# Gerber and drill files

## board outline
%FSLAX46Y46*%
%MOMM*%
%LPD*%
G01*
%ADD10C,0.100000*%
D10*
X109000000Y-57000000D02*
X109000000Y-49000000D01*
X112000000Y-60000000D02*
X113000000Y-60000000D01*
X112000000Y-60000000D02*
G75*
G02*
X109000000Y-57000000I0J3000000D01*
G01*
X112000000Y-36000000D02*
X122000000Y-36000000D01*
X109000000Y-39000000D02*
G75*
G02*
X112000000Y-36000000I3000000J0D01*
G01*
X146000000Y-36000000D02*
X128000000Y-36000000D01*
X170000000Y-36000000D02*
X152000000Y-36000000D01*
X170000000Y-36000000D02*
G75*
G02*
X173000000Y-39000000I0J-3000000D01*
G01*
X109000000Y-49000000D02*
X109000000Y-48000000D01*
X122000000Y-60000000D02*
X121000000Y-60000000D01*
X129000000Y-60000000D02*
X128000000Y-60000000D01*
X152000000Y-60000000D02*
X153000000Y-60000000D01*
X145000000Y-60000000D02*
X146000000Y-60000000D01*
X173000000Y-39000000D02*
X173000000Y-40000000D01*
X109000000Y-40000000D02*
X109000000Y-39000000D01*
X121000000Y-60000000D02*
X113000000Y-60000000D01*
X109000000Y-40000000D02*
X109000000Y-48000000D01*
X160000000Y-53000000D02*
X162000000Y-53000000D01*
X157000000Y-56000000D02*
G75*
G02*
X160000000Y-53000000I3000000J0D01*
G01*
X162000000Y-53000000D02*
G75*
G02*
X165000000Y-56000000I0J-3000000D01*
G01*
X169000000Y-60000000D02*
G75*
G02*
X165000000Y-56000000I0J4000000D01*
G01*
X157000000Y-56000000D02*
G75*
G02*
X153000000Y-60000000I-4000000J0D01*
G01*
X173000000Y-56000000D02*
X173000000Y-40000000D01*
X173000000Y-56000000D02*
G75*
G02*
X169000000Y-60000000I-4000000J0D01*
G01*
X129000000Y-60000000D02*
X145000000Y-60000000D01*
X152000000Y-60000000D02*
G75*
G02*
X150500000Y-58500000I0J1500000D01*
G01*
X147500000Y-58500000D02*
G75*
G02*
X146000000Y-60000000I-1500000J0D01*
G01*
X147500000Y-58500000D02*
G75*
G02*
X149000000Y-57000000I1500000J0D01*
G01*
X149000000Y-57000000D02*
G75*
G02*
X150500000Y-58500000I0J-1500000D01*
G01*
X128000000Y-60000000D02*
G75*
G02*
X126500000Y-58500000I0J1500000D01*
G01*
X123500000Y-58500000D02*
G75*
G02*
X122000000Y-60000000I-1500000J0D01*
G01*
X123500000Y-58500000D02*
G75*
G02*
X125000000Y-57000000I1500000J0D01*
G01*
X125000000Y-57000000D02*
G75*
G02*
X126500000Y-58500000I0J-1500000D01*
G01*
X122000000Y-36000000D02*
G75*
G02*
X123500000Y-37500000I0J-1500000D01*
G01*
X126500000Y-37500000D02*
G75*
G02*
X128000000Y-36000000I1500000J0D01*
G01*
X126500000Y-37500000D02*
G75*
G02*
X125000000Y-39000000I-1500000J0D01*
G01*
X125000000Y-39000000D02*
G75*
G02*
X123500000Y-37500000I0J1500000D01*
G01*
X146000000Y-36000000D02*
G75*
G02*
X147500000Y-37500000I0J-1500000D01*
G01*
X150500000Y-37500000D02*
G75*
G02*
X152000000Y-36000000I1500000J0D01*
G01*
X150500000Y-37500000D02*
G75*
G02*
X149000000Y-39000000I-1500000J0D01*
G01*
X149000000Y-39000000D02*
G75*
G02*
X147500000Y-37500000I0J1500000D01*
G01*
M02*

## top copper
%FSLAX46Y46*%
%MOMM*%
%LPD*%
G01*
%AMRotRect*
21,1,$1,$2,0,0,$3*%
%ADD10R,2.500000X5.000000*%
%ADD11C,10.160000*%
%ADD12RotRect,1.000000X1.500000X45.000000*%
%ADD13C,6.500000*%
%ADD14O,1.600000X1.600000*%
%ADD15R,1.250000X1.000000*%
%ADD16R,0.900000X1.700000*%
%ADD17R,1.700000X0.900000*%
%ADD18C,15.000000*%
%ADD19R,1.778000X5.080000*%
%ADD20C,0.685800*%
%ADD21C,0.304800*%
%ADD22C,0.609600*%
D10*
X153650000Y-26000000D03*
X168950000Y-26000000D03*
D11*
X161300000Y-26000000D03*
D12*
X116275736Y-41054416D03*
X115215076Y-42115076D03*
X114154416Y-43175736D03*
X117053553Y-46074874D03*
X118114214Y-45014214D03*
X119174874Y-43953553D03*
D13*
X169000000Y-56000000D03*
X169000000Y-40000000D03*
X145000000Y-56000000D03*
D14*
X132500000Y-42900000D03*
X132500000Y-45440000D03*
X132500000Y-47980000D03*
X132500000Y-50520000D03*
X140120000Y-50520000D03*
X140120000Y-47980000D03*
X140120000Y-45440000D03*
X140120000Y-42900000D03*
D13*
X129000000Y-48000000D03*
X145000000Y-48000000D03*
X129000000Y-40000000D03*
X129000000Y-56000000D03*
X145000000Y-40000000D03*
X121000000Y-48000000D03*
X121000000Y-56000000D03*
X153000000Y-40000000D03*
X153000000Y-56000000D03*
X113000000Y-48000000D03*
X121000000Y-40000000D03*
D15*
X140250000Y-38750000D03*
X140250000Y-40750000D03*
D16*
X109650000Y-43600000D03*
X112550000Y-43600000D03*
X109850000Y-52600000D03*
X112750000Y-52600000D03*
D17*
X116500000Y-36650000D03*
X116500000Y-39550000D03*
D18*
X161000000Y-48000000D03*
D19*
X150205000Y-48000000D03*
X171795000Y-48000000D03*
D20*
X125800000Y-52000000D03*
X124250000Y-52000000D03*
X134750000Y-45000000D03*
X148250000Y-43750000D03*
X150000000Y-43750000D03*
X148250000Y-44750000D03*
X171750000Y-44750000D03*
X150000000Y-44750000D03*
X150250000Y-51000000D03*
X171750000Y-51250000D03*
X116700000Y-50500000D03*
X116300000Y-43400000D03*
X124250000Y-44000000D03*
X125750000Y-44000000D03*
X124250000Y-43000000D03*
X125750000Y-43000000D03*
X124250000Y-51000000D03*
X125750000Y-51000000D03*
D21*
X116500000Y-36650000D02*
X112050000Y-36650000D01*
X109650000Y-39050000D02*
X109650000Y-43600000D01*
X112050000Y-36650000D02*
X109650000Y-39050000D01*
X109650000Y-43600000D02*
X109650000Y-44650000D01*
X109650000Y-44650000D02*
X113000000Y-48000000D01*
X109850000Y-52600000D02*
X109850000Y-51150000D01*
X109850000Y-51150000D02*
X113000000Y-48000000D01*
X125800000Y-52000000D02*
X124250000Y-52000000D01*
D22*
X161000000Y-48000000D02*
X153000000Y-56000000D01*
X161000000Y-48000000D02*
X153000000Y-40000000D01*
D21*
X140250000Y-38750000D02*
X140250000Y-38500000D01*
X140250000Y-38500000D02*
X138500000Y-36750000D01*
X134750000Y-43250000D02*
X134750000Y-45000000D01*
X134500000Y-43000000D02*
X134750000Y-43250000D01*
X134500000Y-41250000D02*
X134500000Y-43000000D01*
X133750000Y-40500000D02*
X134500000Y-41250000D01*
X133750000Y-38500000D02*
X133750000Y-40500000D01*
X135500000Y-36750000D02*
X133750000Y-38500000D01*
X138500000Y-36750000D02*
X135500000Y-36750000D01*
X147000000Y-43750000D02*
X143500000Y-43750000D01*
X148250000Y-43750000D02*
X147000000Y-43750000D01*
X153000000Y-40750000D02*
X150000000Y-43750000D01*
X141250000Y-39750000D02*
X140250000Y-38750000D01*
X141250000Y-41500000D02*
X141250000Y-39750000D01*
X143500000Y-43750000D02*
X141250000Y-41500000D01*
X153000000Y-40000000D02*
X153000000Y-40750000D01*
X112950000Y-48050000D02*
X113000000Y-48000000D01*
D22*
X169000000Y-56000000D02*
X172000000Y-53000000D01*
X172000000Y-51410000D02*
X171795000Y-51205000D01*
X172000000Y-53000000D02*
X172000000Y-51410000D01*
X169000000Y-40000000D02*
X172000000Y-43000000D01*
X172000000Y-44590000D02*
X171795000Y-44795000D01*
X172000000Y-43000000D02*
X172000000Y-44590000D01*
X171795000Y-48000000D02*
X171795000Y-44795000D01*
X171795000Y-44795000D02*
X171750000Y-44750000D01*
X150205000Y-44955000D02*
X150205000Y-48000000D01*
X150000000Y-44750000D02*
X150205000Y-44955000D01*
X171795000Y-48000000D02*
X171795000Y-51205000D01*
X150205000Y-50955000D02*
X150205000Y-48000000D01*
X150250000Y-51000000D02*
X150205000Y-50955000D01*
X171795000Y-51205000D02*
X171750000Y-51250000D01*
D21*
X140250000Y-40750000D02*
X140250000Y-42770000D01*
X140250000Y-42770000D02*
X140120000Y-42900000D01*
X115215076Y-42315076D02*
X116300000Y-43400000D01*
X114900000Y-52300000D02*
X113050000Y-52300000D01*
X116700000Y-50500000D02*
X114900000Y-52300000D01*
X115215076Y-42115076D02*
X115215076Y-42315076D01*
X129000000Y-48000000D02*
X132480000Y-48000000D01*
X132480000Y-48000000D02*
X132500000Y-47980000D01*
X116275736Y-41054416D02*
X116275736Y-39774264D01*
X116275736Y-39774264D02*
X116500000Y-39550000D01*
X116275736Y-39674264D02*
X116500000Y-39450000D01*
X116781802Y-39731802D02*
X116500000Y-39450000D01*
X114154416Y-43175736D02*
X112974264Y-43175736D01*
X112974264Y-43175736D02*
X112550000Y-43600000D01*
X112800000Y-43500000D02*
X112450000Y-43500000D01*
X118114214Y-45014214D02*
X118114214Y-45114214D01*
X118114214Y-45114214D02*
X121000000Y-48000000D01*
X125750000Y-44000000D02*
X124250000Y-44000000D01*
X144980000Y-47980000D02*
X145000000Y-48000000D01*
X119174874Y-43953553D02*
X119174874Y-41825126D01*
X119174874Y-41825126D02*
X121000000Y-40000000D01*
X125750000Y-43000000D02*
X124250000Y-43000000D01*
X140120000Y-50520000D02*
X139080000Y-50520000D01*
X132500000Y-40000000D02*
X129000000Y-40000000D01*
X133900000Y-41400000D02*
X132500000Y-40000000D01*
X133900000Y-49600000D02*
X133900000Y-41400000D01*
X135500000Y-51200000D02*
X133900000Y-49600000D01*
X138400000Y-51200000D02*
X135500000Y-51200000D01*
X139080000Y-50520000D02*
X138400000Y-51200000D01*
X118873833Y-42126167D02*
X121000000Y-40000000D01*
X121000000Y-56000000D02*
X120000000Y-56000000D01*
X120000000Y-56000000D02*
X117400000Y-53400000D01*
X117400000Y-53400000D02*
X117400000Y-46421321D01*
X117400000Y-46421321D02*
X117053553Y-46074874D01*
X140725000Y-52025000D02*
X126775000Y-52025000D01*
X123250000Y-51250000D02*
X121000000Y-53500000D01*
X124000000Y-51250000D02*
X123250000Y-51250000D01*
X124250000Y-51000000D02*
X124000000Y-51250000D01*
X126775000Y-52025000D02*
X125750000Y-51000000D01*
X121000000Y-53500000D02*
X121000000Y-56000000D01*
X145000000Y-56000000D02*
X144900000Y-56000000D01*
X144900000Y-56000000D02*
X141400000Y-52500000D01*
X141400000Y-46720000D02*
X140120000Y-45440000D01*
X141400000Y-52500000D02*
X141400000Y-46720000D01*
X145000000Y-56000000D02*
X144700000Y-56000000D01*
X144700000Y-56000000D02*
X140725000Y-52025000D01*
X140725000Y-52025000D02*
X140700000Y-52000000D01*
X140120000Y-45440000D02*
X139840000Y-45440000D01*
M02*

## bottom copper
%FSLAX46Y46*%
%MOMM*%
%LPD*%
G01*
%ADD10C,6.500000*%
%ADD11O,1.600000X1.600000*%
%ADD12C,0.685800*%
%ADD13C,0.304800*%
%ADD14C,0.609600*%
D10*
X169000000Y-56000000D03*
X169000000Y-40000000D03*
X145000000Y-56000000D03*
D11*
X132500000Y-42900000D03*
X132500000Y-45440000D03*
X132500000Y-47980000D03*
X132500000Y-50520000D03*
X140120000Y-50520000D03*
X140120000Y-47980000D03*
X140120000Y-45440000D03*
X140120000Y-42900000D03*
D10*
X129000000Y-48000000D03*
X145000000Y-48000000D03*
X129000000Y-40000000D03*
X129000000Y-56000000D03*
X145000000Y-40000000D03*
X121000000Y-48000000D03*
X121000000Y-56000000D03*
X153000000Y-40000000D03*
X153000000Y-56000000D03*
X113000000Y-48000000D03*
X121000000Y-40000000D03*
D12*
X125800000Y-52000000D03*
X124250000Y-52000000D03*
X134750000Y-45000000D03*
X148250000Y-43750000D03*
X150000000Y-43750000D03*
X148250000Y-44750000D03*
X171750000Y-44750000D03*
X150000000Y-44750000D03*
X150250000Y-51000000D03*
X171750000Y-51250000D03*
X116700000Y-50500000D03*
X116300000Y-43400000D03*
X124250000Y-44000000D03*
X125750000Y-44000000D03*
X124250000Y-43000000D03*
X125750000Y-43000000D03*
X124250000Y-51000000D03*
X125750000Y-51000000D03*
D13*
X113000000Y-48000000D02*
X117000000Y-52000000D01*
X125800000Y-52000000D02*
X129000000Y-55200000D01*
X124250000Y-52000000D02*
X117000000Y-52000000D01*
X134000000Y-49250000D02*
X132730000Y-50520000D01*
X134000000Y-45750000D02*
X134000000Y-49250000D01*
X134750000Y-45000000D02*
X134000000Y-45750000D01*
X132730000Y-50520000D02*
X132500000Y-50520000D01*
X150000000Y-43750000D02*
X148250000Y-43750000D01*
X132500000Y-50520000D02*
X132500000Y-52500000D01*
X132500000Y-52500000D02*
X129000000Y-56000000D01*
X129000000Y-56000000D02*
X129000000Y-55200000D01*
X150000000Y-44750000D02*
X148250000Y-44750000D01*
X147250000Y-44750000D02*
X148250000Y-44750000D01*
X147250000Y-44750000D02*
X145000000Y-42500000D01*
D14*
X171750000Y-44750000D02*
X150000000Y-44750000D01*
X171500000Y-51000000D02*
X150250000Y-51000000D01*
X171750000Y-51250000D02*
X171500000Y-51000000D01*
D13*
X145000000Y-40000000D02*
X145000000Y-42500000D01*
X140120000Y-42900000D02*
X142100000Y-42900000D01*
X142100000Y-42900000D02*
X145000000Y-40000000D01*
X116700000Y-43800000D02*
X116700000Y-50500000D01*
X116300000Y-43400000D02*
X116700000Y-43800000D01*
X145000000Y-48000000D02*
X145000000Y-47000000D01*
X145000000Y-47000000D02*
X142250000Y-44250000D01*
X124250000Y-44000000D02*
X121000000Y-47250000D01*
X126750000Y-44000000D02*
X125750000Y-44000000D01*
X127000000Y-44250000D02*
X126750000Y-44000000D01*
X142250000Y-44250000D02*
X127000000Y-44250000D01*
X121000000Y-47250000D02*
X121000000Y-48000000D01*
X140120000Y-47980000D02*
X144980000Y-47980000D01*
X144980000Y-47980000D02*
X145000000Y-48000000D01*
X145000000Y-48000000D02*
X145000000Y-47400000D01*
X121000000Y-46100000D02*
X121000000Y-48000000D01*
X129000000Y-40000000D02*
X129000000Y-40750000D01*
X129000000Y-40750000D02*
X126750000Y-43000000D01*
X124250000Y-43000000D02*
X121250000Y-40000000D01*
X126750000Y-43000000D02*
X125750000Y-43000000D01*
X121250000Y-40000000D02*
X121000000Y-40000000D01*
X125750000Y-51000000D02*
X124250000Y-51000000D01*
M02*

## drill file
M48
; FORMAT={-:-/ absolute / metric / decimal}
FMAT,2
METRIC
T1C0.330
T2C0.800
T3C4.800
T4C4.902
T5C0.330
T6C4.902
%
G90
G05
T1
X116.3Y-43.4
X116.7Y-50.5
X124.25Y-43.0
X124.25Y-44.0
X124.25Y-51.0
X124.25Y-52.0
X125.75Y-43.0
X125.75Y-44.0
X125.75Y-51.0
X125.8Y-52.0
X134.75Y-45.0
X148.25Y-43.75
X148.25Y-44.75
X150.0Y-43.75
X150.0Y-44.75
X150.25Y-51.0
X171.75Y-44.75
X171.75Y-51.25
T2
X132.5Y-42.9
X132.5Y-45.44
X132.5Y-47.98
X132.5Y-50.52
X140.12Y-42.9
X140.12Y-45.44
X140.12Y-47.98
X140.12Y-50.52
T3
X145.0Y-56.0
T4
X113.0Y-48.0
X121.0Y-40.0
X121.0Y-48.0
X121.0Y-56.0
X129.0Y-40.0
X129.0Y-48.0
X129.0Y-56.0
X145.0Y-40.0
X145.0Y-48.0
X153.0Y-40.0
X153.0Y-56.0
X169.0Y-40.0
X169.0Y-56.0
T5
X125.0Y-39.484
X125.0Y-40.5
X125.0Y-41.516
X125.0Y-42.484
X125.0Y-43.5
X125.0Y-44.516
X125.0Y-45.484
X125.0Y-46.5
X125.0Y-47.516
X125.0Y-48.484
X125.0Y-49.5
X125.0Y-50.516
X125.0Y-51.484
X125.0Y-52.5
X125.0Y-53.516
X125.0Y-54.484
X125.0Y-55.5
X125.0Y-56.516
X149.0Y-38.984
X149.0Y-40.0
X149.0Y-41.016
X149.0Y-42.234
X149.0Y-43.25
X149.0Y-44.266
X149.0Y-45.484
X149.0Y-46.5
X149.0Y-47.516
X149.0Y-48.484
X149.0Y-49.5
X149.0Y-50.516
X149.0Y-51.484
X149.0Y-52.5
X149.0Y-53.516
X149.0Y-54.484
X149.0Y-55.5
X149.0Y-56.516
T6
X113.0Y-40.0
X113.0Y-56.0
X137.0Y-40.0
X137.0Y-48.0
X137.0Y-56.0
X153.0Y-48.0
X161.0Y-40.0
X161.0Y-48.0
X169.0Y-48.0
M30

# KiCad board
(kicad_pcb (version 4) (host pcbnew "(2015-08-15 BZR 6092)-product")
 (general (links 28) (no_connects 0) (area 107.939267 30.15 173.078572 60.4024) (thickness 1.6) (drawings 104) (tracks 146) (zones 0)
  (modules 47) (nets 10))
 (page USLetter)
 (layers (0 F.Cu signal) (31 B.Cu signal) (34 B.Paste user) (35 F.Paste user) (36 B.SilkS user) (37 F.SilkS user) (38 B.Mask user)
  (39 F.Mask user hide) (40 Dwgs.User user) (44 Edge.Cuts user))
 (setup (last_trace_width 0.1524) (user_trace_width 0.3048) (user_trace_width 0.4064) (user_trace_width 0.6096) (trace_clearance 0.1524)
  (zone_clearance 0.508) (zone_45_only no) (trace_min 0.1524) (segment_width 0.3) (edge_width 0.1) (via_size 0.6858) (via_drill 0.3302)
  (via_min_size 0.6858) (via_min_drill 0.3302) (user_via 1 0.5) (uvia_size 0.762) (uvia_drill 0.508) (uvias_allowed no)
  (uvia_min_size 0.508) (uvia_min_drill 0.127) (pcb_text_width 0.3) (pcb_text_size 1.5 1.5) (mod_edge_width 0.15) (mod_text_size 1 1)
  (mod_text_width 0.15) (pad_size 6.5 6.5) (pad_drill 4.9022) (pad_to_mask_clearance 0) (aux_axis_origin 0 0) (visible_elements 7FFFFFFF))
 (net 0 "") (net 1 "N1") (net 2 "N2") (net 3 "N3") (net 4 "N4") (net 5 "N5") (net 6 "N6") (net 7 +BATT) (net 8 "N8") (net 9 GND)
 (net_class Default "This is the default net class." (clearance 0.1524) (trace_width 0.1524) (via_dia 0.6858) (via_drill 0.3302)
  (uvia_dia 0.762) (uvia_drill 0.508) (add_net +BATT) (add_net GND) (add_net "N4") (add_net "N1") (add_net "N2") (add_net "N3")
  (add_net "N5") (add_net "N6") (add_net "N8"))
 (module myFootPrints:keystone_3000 (layer F.Cu) (at 161.3 26)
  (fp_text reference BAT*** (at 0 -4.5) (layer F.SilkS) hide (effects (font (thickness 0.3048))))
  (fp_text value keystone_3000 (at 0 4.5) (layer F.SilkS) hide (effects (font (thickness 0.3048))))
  (pad 1 smd rect (at -7.65 0) (size 2.5 5) (layers F.Cu F.Paste F.Mask))
  (pad 1 smd rect (at 7.65 0) (size 2.5 5) (layers F.Cu F.Paste F.Mask))
  (pad 2 smd circle (at 0 0) (size 10.16 10.16) (layers F.Cu F.Paste F.Mask)))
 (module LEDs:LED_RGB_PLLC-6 (layer F.Cu) (at 116.7 43.6 315)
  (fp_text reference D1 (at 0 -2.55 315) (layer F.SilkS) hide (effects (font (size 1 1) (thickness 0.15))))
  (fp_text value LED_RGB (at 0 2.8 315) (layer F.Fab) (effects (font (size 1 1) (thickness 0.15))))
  (pad 1 smd rect (at -2.1 -1.5 45) (size 1 1.5) (layers F.Cu F.Paste F.Mask) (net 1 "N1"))
  (pad 2 smd rect (at -2.1 0 45) (size 1 1.5) (layers F.Cu F.Paste F.Mask) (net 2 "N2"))
  (pad 3 smd rect (at -2.1 1.5 45) (size 1 1.5) (layers F.Cu F.Paste F.Mask) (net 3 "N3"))
  (pad 4 smd rect (at 2 1.5 45) (size 1 1.5) (layers F.Cu F.Paste F.Mask) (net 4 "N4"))
  (pad 5 smd rect (at 2 0 45) (size 1 1.5) (layers F.Cu F.Paste F.Mask) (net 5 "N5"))
  (pad 6 smd rect (at 2 -1.5 45) (size 1 1.5) (layers F.Cu F.Paste F.Mask) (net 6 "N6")))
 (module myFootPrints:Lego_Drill (layer F.Cu) (at 113 40)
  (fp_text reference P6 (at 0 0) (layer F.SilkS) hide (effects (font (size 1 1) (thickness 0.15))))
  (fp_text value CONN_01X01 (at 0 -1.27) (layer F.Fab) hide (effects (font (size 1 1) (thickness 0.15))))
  (pad "" np_thru_hole circle (at 0 0) (size 4.9022 4.9022) (drill 4.9022) (layers *.Cu *.Mask F.SilkS)))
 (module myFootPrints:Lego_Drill (layer F.Cu) (at 113 56)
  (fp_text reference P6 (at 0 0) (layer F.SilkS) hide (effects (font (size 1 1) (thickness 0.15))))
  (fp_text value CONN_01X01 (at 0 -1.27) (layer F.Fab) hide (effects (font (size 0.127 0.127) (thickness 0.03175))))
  (pad "" np_thru_hole circle (at 0 0) (size 4.9022 4.9022) (drill 4.9022) (layers *.Cu *.Mask F.SilkS)))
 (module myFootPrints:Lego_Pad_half (layer F.Cu) (at 169 56 180)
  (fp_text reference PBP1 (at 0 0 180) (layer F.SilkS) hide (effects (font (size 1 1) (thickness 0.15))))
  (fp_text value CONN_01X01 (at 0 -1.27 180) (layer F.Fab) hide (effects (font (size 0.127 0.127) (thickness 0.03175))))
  (pad 1 thru_hole circle (at 0 0 180) (size 6.5 6.5) (drill 4.9022) (layers *.Cu B.Mask) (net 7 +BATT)))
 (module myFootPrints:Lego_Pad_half (layer F.Cu) (at 169 40 270)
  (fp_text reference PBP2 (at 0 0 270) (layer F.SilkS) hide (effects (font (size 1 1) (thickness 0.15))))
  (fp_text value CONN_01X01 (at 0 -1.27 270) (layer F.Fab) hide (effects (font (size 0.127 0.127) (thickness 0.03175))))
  (pad 1 thru_hole circle (at 0 0 270) (size 6.5 6.5) (drill 4.9022) (layers *.Cu B.Mask) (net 7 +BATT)))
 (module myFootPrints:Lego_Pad (layer F.Cu) (at 145 56)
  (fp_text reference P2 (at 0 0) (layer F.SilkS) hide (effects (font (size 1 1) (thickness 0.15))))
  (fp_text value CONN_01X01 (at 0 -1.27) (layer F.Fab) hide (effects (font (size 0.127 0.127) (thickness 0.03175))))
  (pad 1 thru_hole circle (at 0 0) (size 6.5 6.5) (drill 4.8) (layers *.Cu *.Mask F.SilkS) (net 4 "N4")))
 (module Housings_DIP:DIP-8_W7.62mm (layer F.Cu) (at 132.5 42.9)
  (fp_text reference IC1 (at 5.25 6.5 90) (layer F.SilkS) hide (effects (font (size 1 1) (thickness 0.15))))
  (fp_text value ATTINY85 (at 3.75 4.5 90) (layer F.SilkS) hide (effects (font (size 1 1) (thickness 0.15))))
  (pad 1 thru_hole oval (at 0 0) (size 1.6 1.6) (drill 0.8) (layers *.Cu *.Mask F.SilkS))
  (pad 2 thru_hole oval (at 0 2.54) (size 1.6 1.6) (drill 0.8) (layers *.Cu *.Mask F.SilkS))
  (pad 3 thru_hole oval (at 0 5.08) (size 1.6 1.6) (drill 0.8) (layers *.Cu *.Mask F.SilkS) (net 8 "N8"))
  (pad 4 thru_hole oval (at 0 7.62) (size 1.6 1.6) (drill 0.8) (layers *.Cu *.Mask F.SilkS) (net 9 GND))
  (pad 5 thru_hole oval (at 7.62 7.62) (size 1.6 1.6) (drill 0.8) (layers *.Cu *.Mask F.SilkS) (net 6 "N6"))
  (pad 6 thru_hole oval (at 7.62 5.08) (size 1.6 1.6) (drill 0.8) (layers *.Cu *.Mask F.SilkS) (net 5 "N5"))
  (pad 7 thru_hole oval (at 7.62 2.54) (size 1.6 1.6) (drill 0.8) (layers *.Cu *.Mask F.SilkS) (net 4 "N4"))
  (pad 8 thru_hole oval (at 7.62 0) (size 1.6 1.6) (drill 0.8) (layers *.Cu *.Mask F.SilkS) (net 7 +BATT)))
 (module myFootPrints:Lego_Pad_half (layer F.Cu) (at 129 48 45)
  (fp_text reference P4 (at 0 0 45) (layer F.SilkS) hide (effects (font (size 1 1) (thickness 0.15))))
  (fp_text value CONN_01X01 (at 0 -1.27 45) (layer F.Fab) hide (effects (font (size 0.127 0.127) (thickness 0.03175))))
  (pad 1 thru_hole circle (at 0 0 45) (size 6.5 6.5) (drill 4.9022) (layers *.Cu *.Mask F.SilkS) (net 8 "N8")))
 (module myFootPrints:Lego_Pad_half (layer F.Cu) (at 145 48 225)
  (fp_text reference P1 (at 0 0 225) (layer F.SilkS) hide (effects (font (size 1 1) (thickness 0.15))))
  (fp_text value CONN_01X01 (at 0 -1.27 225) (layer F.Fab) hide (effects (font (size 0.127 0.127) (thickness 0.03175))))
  (pad 1 thru_hole circle (at 0 0 225) (size 6.5 6.5) (drill 4.9022) (layers *.Cu *.Mask F.SilkS) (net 5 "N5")))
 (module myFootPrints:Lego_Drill (layer F.Cu) (at 137 40)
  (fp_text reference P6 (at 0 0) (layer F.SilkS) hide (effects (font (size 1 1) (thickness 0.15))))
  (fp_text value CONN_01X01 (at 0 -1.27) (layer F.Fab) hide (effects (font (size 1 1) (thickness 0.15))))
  (pad "" np_thru_hole circle (at 0 0) (size 4.9022 4.9022) (drill 4.9022) (layers *.Cu *.Mask F.SilkS)))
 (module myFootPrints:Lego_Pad (layer F.Cu) (at 129 40)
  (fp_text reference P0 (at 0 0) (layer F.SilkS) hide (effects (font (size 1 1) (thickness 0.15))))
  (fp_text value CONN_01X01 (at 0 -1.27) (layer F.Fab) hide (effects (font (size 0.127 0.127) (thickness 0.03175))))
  (pad 1 thru_hole circle (at 0 0) (size 6.5 6.5) (drill 4.9022) (layers *.Cu *.Mask F.SilkS) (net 6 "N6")))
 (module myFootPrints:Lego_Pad (layer F.Cu) (at 129 56)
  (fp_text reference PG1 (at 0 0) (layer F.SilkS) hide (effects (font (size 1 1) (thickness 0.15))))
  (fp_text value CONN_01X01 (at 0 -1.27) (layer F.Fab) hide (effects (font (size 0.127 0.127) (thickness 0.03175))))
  (pad 1 thru_hole circle (at 0 0) (size 6.5 6.5) (drill 4.9022) (layers *.Cu *.Mask F.SilkS) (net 9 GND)))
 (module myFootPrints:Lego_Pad (layer F.Cu) (at 145 40)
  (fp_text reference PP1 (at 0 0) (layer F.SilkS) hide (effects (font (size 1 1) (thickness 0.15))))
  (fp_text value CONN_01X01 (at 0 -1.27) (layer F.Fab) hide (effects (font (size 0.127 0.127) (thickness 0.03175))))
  (pad 1 thru_hole circle (at 0 0) (size 6.5 6.5) (drill 4.9022) (layers *.Cu *.Mask F.SilkS) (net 7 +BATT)))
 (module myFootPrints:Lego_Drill (layer F.Cu) (at 137 48)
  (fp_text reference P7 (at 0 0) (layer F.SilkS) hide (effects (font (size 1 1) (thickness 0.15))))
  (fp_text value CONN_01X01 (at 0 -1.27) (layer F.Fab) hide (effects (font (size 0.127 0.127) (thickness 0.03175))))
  (pad "" np_thru_hole circle (at 0 0) (size 4.9022 4.9022) (drill 4.9022) (layers *.Cu *.Mask F.SilkS)))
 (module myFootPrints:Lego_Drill (layer F.Cu) (at 137 56)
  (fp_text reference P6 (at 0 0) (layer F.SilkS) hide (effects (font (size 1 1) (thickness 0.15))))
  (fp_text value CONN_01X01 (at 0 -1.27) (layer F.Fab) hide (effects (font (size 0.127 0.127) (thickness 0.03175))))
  (pad "" np_thru_hole circle (at 0 0) (size 4.9022 4.9022) (drill 4.9022) (layers *.Cu *.Mask F.SilkS)))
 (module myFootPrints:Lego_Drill (layer F.Cu) (at 161 48)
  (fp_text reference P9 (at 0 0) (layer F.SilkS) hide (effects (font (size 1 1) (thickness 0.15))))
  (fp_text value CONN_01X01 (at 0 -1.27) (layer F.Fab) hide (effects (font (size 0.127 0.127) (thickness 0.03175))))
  (pad "" np_thru_hole circle (at 0 0) (size 4.9022 4.9022) (drill 4.9022) (layers *.Cu *.Mask F.SilkS)))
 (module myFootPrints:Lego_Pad (layer F.Cu) (at 121 48)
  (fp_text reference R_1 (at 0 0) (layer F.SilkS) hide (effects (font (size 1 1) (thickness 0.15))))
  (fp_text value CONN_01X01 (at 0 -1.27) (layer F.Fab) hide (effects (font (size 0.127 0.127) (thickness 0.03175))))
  (pad 1 thru_hole circle (at 0 0) (size 6.5 6.5) (drill 4.9022) (layers *.Cu *.Mask F.SilkS) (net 5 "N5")))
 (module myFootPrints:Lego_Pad (layer F.Cu) (at 121 56)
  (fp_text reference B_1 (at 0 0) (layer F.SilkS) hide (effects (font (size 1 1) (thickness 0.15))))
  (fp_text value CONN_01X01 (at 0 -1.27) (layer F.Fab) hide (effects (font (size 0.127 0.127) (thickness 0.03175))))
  (pad 1 thru_hole circle (at 0 0) (size 6.5 6.5) (drill 4.9022) (layers *.Cu *.Mask F.SilkS) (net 4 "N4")))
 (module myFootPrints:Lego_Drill (layer F.Cu) (at 169 48)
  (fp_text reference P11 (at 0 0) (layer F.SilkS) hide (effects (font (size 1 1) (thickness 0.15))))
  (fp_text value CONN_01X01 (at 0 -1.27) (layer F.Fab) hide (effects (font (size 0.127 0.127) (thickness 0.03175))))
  (pad "" np_thru_hole circle (at 0 0) (size 4.9022 4.9022) (drill 4.9022) (layers *.Cu *.Mask F.SilkS)))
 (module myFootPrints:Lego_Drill (layer F.Cu) (at 153 48)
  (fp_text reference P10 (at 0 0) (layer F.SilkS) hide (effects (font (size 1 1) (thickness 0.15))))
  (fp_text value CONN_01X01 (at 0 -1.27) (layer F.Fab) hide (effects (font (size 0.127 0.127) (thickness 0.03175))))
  (pad "" np_thru_hole circle (at 0 0) (size 4.9022 4.9022) (drill 4.9022) (layers *.Cu *.Mask F.SilkS)))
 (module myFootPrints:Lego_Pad (layer F.Cu) (at 153 40)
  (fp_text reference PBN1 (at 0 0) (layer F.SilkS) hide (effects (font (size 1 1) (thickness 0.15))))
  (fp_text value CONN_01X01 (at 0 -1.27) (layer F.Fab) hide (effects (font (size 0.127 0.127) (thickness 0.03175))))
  (pad 1 thru_hole circle (at 0 0) (size 6.5 6.5) (drill 4.9022) (layers *.Cu *.Mask F.SilkS) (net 9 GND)))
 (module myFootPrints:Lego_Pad (layer F.Cu) (at 153 56)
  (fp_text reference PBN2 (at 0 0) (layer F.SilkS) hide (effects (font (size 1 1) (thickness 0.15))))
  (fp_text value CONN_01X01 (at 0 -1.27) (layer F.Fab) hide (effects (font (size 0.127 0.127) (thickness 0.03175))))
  (pad 1 thru_hole circle (at 0 0) (size 6.5 6.5) (drill 4.9022) (layers *.Cu *.Mask F.SilkS) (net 9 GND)))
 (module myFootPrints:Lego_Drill (layer F.Cu) (at 161 40)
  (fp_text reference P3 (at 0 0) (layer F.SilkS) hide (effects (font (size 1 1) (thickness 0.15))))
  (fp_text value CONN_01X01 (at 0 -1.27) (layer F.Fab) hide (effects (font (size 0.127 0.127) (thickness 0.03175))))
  (pad "" np_thru_hole circle (at 0 0) (size 4.9022 4.9022) (drill 4.9022) (layers *.Cu *.Mask F.SilkS)))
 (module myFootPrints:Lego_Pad (layer F.Cu) (at 113 48)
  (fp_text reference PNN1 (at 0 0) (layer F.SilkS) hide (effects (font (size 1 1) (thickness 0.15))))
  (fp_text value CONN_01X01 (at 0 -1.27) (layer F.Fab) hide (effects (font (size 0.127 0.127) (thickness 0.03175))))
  (pad 1 thru_hole circle (at 0 0) (size 6.5 6.5) (drill 4.9022) (layers *.Cu *.Mask F.SilkS) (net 9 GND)))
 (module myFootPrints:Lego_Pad (layer F.Cu) (at 121 40)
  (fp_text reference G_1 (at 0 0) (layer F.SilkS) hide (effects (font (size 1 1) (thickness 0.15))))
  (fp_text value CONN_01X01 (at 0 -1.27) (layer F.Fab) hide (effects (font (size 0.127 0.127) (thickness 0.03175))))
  (pad 1 thru_hole circle (at 0 0) (size 6.5 6.5) (drill 4.9022) (layers *.Cu *.Mask F.SilkS) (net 6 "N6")))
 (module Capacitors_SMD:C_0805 (layer F.Cu) (at 140.25 39.75 270)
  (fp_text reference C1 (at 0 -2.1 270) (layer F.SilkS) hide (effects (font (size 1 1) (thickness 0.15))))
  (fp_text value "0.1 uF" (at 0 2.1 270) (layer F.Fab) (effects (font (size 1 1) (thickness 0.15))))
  (pad 1 smd rect (at -1 0 270) (size 1 1.25) (layers F.Cu F.Paste F.Mask) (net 9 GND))
  (pad 2 smd rect (at 1 0 270) (size 1 1.25) (layers F.Cu F.Paste F.Mask) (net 7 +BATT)))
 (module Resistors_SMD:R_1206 (layer F.Cu) (at 111.1 43.6)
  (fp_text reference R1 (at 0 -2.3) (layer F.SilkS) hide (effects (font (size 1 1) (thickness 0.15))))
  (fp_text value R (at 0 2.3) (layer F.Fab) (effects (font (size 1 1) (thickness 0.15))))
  (pad 1 smd rect (at -1.45 0) (size 0.9 1.7) (layers F.Cu F.Paste F.Mask) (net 9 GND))
  (pad 2 smd rect (at 1.45 0) (size 0.9 1.7) (layers F.Cu F.Paste F.Mask) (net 3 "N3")))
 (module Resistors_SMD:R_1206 (layer F.Cu) (at 111.3 52.6)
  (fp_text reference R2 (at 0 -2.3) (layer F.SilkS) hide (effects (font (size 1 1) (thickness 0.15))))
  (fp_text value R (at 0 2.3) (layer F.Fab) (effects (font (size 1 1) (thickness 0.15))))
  (pad 1 smd rect (at -1.45 0) (size 0.9 1.7) (layers F.Cu F.Paste F.Mask) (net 9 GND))
  (pad 2 smd rect (at 1.45 0) (size 0.9 1.7) (layers F.Cu F.Paste F.Mask) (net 2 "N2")))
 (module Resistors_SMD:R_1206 (layer F.Cu) (at 116.5 38.1 270)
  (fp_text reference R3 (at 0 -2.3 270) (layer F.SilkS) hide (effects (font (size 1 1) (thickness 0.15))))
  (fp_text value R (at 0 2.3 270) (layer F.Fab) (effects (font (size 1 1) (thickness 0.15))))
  (pad 1 smd rect (at -1.45 0 270) (size 0.9 1.7) (layers F.Cu F.Paste F.Mask) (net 9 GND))
  (pad 2 smd rect (at 1.45 0 270) (size 0.9 1.7) (layers F.Cu F.Paste F.Mask) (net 1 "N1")))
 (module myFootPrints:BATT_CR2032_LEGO (layer F.Cu) (at 161 48)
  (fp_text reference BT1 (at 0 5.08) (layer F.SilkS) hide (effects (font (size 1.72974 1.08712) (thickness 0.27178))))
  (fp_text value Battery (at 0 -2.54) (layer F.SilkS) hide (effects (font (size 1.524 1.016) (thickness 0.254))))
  (pad 2 smd circle (at 0 0) (size 15 15) (layers F.Cu F.Paste F.Mask) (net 9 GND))
  (pad 1 smd rect (at -10.795 0) (size 1.778 5.08) (layers F.Cu F.Paste F.Mask) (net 7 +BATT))
  (pad 1 smd rect (at 10.795 0) (size 1.778 5.08) (layers F.Cu F.Paste F.Mask) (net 7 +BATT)))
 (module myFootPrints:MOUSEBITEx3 (layer F.Cu) (at 149 40 90)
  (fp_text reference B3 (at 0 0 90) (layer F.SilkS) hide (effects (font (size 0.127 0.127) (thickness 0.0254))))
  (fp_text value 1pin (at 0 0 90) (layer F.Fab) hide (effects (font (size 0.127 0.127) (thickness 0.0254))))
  (pad "" np_thru_hole circle (at -1.016 0 90) (size 0.3302 0.3302) (drill 0.3302) (layers *.Cu *.Mask F.SilkS))
  (pad "" np_thru_hole circle (at 1.016 0 90) (size 0.3302 0.3302) (drill 0.3302) (layers *.Cu *.Mask F.SilkS))
  (pad "" np_thru_hole circle (at 0 0 90) (size 0.3302 0.3302) (drill 0.3302) (layers *.Cu *.Mask F.SilkS)))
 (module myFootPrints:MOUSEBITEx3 (layer F.Cu) (at 149 49.5 90)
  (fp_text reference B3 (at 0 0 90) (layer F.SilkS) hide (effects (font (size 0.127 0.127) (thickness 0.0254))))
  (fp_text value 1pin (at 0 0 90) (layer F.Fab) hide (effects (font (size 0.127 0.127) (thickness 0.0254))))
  (pad "" np_thru_hole circle (at -1.016 0 90) (size 0.3302 0.3302) (drill 0.3302) (layers *.Cu *.Mask F.SilkS))
  (pad "" np_thru_hole circle (at 1.016 0 90) (size 0.3302 0.3302) (drill 0.3302) (layers *.Cu *.Mask F.SilkS))
  (pad "" np_thru_hole circle (at 0 0 90) (size 0.3302 0.3302) (drill 0.3302) (layers *.Cu *.Mask F.SilkS)))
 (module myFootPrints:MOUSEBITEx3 (layer F.Cu) (at 149 52.5 90)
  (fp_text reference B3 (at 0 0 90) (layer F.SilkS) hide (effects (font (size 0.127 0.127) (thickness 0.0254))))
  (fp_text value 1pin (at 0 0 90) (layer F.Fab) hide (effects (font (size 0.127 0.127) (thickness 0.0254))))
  (pad "" np_thru_hole circle (at -1.016 0 90) (size 0.3302 0.3302) (drill 0.3302) (layers *.Cu *.Mask F.SilkS))
  (pad "" np_thru_hole circle (at 1.016 0 90) (size 0.3302 0.3302) (drill 0.3302) (layers *.Cu *.Mask F.SilkS))
  (pad "" np_thru_hole circle (at 0 0 90) (size 0.3302 0.3302) (drill 0.3302) (layers *.Cu *.Mask F.SilkS)))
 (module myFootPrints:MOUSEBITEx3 (layer F.Cu) (at 149 55.5 90)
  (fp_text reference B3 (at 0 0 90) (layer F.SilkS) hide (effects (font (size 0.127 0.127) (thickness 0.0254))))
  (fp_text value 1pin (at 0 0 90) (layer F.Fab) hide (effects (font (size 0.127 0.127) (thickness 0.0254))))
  (pad "" np_thru_hole circle (at -1.016 0 90) (size 0.3302 0.3302) (drill 0.3302) (layers *.Cu *.Mask F.SilkS))
  (pad "" np_thru_hole circle (at 1.016 0 90) (size 0.3302 0.3302) (drill 0.3302) (layers *.Cu *.Mask F.SilkS))
  (pad "" np_thru_hole circle (at 0 0 90) (size 0.3302 0.3302) (drill 0.3302) (layers *.Cu *.Mask F.SilkS)))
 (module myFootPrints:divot (layer F.Cu) (at 149 60 180)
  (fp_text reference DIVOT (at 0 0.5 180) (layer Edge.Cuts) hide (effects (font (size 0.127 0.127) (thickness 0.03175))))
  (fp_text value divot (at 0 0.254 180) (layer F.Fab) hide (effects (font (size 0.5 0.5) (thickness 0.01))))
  (fp_arc (start -3 1.5) (end -3 0) (angle 90) (layer Edge.Cuts) (width 0.1))
  (fp_arc (start 3 1.5) (end 1.5 1.5) (angle 90) (layer Edge.Cuts) (width 0.1))
  (fp_arc (start 0 1.5) (end 1.5 1.5) (angle 90) (layer Edge.Cuts) (width 0.1))
  (fp_arc (start 0 1.5) (end 0 3) (angle 90) (layer Edge.Cuts) (width 0.1)))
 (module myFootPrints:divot (layer F.Cu) (at 125 60 180)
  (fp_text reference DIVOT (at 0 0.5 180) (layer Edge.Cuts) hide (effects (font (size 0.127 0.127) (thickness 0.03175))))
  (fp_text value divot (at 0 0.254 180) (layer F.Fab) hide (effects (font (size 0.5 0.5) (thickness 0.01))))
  (fp_arc (start -3 1.5) (end -3 0) (angle 90) (layer Edge.Cuts) (width 0.1))
  (fp_arc (start 3 1.5) (end 1.5 1.5) (angle 90) (layer Edge.Cuts) (width 0.1))
  (fp_arc (start 0 1.5) (end 1.5 1.5) (angle 90) (layer Edge.Cuts) (width 0.1))
  (fp_arc (start 0 1.5) (end 0 3) (angle 90) (layer Edge.Cuts) (width 0.1)))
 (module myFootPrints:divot (layer F.Cu) (at 125 36)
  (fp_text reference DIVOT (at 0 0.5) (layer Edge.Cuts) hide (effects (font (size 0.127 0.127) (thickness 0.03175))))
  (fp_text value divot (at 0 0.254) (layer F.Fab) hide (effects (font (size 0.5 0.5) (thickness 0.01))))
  (fp_arc (start -3 1.5) (end -3 0) (angle 90) (layer Edge.Cuts) (width 0.1))
  (fp_arc (start 3 1.5) (end 1.5 1.5) (angle 90) (layer Edge.Cuts) (width 0.1))
  (fp_arc (start 0 1.5) (end 1.5 1.5) (angle 90) (layer Edge.Cuts) (width 0.1))
  (fp_arc (start 0 1.5) (end 0 3) (angle 90) (layer Edge.Cuts) (width 0.1)))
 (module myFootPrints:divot (layer F.Cu) (at 149 36)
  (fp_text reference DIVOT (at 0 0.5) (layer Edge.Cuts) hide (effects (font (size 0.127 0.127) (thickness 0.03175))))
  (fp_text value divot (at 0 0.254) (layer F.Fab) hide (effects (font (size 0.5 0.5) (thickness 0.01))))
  (fp_arc (start -3 1.5) (end -3 0) (angle 90) (layer Edge.Cuts) (width 0.1))
  (fp_arc (start 3 1.5) (end 1.5 1.5) (angle 90) (layer Edge.Cuts) (width 0.1))
  (fp_arc (start 0 1.5) (end 1.5 1.5) (angle 90) (layer Edge.Cuts) (width 0.1))
  (fp_arc (start 0 1.5) (end 0 3) (angle 90) (layer Edge.Cuts) (width 0.1)))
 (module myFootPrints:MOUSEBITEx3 (layer F.Cu) (at 149 46.5 90)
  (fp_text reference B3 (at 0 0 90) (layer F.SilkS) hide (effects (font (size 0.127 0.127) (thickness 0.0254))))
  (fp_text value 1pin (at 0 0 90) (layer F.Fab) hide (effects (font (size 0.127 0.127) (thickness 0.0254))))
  (pad "" np_thru_hole circle (at -1.016 0 90) (size 0.3302 0.3302) (drill 0.3302) (layers *.Cu *.Mask F.SilkS))
  (pad "" np_thru_hole circle (at 1.016 0 90) (size 0.3302 0.3302) (drill 0.3302) (layers *.Cu *.Mask F.SilkS))
  (pad "" np_thru_hole circle (at 0 0 90) (size 0.3302 0.3302) (drill 0.3302) (layers *.Cu *.Mask F.SilkS)))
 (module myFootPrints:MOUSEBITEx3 (layer F.Cu) (at 149 43.25 90)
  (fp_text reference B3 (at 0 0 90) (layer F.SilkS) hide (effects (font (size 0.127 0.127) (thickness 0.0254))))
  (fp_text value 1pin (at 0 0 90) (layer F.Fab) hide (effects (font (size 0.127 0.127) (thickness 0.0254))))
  (pad "" np_thru_hole circle (at -1.016 0 90) (size 0.3302 0.3302) (drill 0.3302) (layers *.Cu *.Mask F.SilkS))
  (pad "" np_thru_hole circle (at 1.016 0 90) (size 0.3302 0.3302) (drill 0.3302) (layers *.Cu *.Mask F.SilkS))
  (pad "" np_thru_hole circle (at 0 0 90) (size 0.3302 0.3302) (drill 0.3302) (layers *.Cu *.Mask F.SilkS)))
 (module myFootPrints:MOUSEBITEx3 (layer F.Cu) (at 125 55.5 90)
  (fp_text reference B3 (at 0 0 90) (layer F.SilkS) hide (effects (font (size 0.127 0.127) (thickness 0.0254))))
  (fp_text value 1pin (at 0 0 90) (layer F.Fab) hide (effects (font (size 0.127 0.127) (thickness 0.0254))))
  (pad "" np_thru_hole circle (at -1.016 0 90) (size 0.3302 0.3302) (drill 0.3302) (layers *.Cu *.Mask F.SilkS))
  (pad "" np_thru_hole circle (at 1.016 0 90) (size 0.3302 0.3302) (drill 0.3302) (layers *.Cu *.Mask F.SilkS))
  (pad "" np_thru_hole circle (at 0 0 90) (size 0.3302 0.3302) (drill 0.3302) (layers *.Cu *.Mask F.SilkS)))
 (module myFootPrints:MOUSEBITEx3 (layer F.Cu) (at 125 52.5 90)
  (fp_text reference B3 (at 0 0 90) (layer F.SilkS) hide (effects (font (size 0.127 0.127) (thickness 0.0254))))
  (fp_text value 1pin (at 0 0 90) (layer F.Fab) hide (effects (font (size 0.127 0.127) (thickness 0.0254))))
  (pad "" np_thru_hole circle (at -1.016 0 90) (size 0.3302 0.3302) (drill 0.3302) (layers *.Cu *.Mask F.SilkS))
  (pad "" np_thru_hole circle (at 1.016 0 90) (size 0.3302 0.3302) (drill 0.3302) (layers *.Cu *.Mask F.SilkS))
  (pad "" np_thru_hole circle (at 0 0 90) (size 0.3302 0.3302) (drill 0.3302) (layers *.Cu *.Mask F.SilkS)))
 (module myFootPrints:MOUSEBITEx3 (layer F.Cu) (at 125 49.5 90)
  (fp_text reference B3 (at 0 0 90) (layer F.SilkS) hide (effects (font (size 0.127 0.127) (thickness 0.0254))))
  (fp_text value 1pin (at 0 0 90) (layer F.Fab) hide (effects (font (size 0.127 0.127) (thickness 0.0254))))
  (pad "" np_thru_hole circle (at -1.016 0 90) (size 0.3302 0.3302) (drill 0.3302) (layers *.Cu *.Mask F.SilkS))
  (pad "" np_thru_hole circle (at 1.016 0 90) (size 0.3302 0.3302) (drill 0.3302) (layers *.Cu *.Mask F.SilkS))
  (pad "" np_thru_hole circle (at 0 0 90) (size 0.3302 0.3302) (drill 0.3302) (layers *.Cu *.Mask F.SilkS)))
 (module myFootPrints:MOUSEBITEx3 (layer F.Cu) (at 125 46.5 90)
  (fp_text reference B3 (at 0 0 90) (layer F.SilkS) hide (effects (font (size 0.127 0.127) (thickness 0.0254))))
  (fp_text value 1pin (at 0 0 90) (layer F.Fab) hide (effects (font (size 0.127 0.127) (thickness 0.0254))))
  (pad "" np_thru_hole circle (at -1.016 0 90) (size 0.3302 0.3302) (drill 0.3302) (layers *.Cu *.Mask F.SilkS))
  (pad "" np_thru_hole circle (at 1.016 0 90) (size 0.3302 0.3302) (drill 0.3302) (layers *.Cu *.Mask F.SilkS))
  (pad "" np_thru_hole circle (at 0 0 90) (size 0.3302 0.3302) (drill 0.3302) (layers *.Cu *.Mask F.SilkS)))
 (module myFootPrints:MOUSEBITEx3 (layer F.Cu) (at 125 43.5 90)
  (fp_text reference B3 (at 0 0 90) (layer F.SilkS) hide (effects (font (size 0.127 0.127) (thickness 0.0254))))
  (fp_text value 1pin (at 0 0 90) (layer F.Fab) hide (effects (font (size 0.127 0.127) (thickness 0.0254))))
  (pad "" np_thru_hole circle (at -1.016 0 90) (size 0.3302 0.3302) (drill 0.3302) (layers *.Cu *.Mask F.SilkS))
  (pad "" np_thru_hole circle (at 1.016 0 90) (size 0.3302 0.3302) (drill 0.3302) (layers *.Cu *.Mask F.SilkS))
  (pad "" np_thru_hole circle (at 0 0 90) (size 0.3302 0.3302) (drill 0.3302) (layers *.Cu *.Mask F.SilkS)))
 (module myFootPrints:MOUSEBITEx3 (layer F.Cu) (at 125 40.5 90)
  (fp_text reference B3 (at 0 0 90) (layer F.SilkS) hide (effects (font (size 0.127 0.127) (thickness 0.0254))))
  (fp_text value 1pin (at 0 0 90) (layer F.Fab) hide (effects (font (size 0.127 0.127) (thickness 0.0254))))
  (pad "" np_thru_hole circle (at -1.016 0 90) (size 0.3302 0.3302) (drill 0.3302) (layers *.Cu *.Mask F.SilkS))
  (pad "" np_thru_hole circle (at 1.016 0 90) (size 0.3302 0.3302) (drill 0.3302) (layers *.Cu *.Mask F.SilkS))
  (pad "" np_thru_hole circle (at 0 0 90) (size 0.3302 0.3302) (drill 0.3302) (layers *.Cu *.Mask F.SilkS)))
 (gr_line (start 109 57) (end 109 49) (angle 90) (layer Edge.Cuts) (width 0.1))
 (gr_line (start 112 60) (end 113 60) (angle 90) (layer Edge.Cuts) (width 0.1))
 (gr_arc (start 112 57) (end 112 60) (angle 90) (layer Edge.Cuts) (width 0.1))
 (gr_line (start 112 36) (end 122 36) (angle 90) (layer Edge.Cuts) (width 0.1))
 (gr_arc (start 112 39) (end 109 39) (angle 90) (layer Edge.Cuts) (width 0.1))
 (gr_line (start 146 36) (end 128 36) (angle 90) (layer Edge.Cuts) (width 0.1))
 (gr_line (start 170 36) (end 152 36) (angle 90) (layer Edge.Cuts) (width 0.1))
 (gr_arc (start 170 39) (end 170 36) (angle 90) (layer Edge.Cuts) (width 0.1))
 (gr_line (start 109 49) (end 109 48) (angle 90) (layer Edge.Cuts) (width 0.1))
 (gr_line (start 122 60) (end 121 60) (angle 90) (layer Edge.Cuts) (width 0.1))
 (gr_line (start 129 60) (end 128 60) (angle 90) (layer Edge.Cuts) (width 0.1))
 (gr_line (start 152 60) (end 153 60) (angle 90) (layer Edge.Cuts) (width 0.1))
 (gr_line (start 145 60) (end 146 60) (angle 90) (layer Edge.Cuts) (width 0.1))
 (gr_line (start 173 39) (end 173 40) (angle 90) (layer Edge.Cuts) (width 0.1))
 (gr_line (start 109 40) (end 109 39) (angle 90) (layer Edge.Cuts) (width 0.1))
 (gr_line (start 121 60) (end 113 60) (angle 90) (layer Edge.Cuts) (width 0.1))
 (gr_line (start 109 40) (end 109 48) (angle 90) (layer Edge.Cuts) (width 0.1))
 (gr_line (start 160 53) (end 162 53) (angle 90) (layer Edge.Cuts) (width 0.1))
 (gr_arc (start 160 56) (end 157 56) (angle 90) (layer Edge.Cuts) (width 0.1))
 (gr_arc (start 162 56) (end 162 53) (angle 90) (layer Edge.Cuts) (width 0.1))
 (gr_arc (start 169 56) (end 169 60) (angle 90) (layer Edge.Cuts) (width 0.1))
 (gr_arc (start 153 56) (end 157 56) (angle 90) (layer Edge.Cuts) (width 0.1))
 (gr_line (start 173 56) (end 173 40) (angle 90) (layer Edge.Cuts) (width 0.1))
 (gr_arc (start 169 56) (end 173 56) (angle 90) (layer Edge.Cuts) (width 0.1))
 (gr_line (start 129 60) (end 145 60) (angle 90) (layer Edge.Cuts) (width 0.1))
 (segment (start 116.5 36.65) (end 112.05 36.65) (width 0.3048) (layer F.Cu) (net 9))
 (segment (start 109.65 39.05) (end 109.65 43.6) (width 0.3048) (layer F.Cu) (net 9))
 (segment (start 112.05 36.65) (end 109.65 39.05) (width 0.3048) (layer F.Cu) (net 9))
 (segment (start 109.65 43.6) (end 109.65 44.65) (width 0.3048) (layer F.Cu) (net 9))
 (segment (start 109.65 44.65) (end 113 48) (width 0.3048) (layer F.Cu) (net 9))
 (segment (start 109.85 52.6) (end 109.85 51.15) (width 0.3048) (layer F.Cu) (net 9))
 (segment (start 109.85 51.15) (end 113 48) (width 0.3048) (layer F.Cu) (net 9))
 (via (at 125.8 52) (size 0.6858) (drill 0.3302) (layers F.Cu B.Cu) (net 9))
 (segment (start 113 48) (end 117 52) (width 0.3048) (layer B.Cu) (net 9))
 (segment (start 125.8 52) (end 129 55.2) (width 0.3048) (layer B.Cu) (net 9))
 (segment (start 124.25 52) (end 117 52) (width 0.3048) (layer B.Cu) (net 9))
 (via (at 124.25 52) (size 0.6858) (drill 0.3302) (layers F.Cu B.Cu) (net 9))
 (segment (start 125.8 52) (end 124.25 52) (width 0.3048) (layer F.Cu) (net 9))
 (segment (start 161 48) (end 153 56) (width 0.6096) (layer F.Cu) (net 9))
 (segment (start 161 48) (end 153 40) (width 0.6096) (layer F.Cu) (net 9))
 (segment (start 140.25 38.75) (end 140.25 38.5) (width 0.3048) (layer F.Cu) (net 9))
 (segment (start 140.25 38.5) (end 138.5 36.75) (width 0.3048) (layer F.Cu) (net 9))
 (segment (start 134 49.25) (end 132.73 50.52) (width 0.3048) (layer B.Cu) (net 9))
 (segment (start 134 45.75) (end 134 49.25) (width 0.3048) (layer B.Cu) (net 9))
 (segment (start 134.75 45) (end 134 45.75) (width 0.3048) (layer B.Cu) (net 9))
 (via (at 134.75 45) (size 0.6858) (drill 0.3302) (layers F.Cu B.Cu) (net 9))
 (segment (start 134.75 43.25) (end 134.75 45) (width 0.3048) (layer F.Cu) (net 9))
 (segment (start 134.5 43) (end 134.75 43.25) (width 0.3048) (layer F.Cu) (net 9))
 (segment (start 134.5 41.25) (end 134.5 43) (width 0.3048) (layer F.Cu) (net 9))
 (segment (start 133.75 40.5) (end 134.5 41.25) (width 0.3048) (layer F.Cu) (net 9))
 (segment (start 133.75 38.5) (end 133.75 40.5) (width 0.3048) (layer F.Cu) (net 9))
 (segment (start 135.5 36.75) (end 133.75 38.5) (width 0.3048) (layer F.Cu) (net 9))
 (segment (start 138.5 36.75) (end 135.5 36.75) (width 0.3048) (layer F.Cu) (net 9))
 (segment (start 132.73 50.52) (end 132.5 50.52) (width 0.3048) (layer B.Cu) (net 9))
 (segment (start 147 43.75) (end 143.5 43.75) (width 0.3048) (layer F.Cu) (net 9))
 (segment (start 148.25 43.75) (end 147 43.75) (width 0.3048) (layer F.Cu) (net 9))
 (via (at 148.25 43.75) (size 0.6858) (drill 0.3302) (layers F.Cu B.Cu) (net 9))
 (segment (start 150 43.75) (end 148.25 43.75) (width 0.3048) (layer B.Cu) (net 9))
 (via (at 150 43.75) (size 0.6858) (drill 0.3302) (layers F.Cu B.Cu) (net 9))
 (segment (start 153 40.75) (end 150 43.75) (width 0.3048) (layer F.Cu) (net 9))
 (segment (start 141.25 39.75) (end 140.25 38.75) (width 0.3048) (layer F.Cu) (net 9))
 (segment (start 141.25 41.5) (end 141.25 39.75) (width 0.3048) (layer F.Cu) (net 9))
 (segment (start 143.5 43.75) (end 141.25 41.5) (width 0.3048) (layer F.Cu) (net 9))
 (segment (start 153 40) (end 153 40.75) (width 0.3048) (layer F.Cu) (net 9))
 (segment (start 132.5 50.52) (end 132.5 52.5) (width 0.3048) (layer B.Cu) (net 9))
 (segment (start 132.5 52.5) (end 129 56) (width 0.3048) (layer B.Cu) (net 9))
 (segment (start 129 56) (end 129 55.2) (width 0.3048) (layer B.Cu) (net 9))
 (segment (start 112.95 48.05) (end 113 48) (width 0.3048) (layer F.Cu) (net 9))
 (segment (start 169 56) (end 172 53) (width 0.6096) (layer F.Cu) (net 7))
 (segment (start 172 51.41) (end 171.795 51.205) (width 0.6096) (layer F.Cu) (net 7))
 (segment (start 172 53) (end 172 51.41) (width 0.6096) (layer F.Cu) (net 7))
 (segment (start 169 40) (end 172 43) (width 0.6096) (layer F.Cu) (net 7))
 (segment (start 172 44.59) (end 171.795 44.795) (width 0.6096) (layer F.Cu) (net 7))
 (segment (start 172 43) (end 172 44.59) (width 0.6096) (layer F.Cu) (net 7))
 (segment (start 150 44.75) (end 148.25 44.75) (width 0.3048) (layer B.Cu) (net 7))
 (via (at 148.25 44.75) (size 0.6858) (drill 0.3302) (layers F.Cu B.Cu) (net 7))
 (segment (start 147.25 44.75) (end 148.25 44.75) (width 0.3048) (layer B.Cu) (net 7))
 (segment (start 147.25 44.75) (end 145 42.5) (width 0.3048) (layer B.Cu) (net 7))
 (segment (start 171.795 48) (end 171.795 44.795) (width 0.6096) (layer F.Cu) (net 7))
 (segment (start 171.75 44.75) (end 150 44.75) (width 0.6096) (layer B.Cu) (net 7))
 (via (at 171.75 44.75) (size 0.6858) (drill 0.3302) (layers F.Cu B.Cu) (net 7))
 (segment (start 171.795 44.795) (end 171.75 44.75) (width 0.6096) (layer F.Cu) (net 7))
 (via (at 150 44.75) (size 0.6858) (drill 0.3302) (layers F.Cu B.Cu) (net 7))
 (segment (start 150.205 44.955) (end 150.205 48) (width 0.6096) (layer F.Cu) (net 7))
 (segment (start 150 44.75) (end 150.205 44.955) (width 0.6096) (layer F.Cu) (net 7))
 (segment (start 171.795 48) (end 171.795 51.205) (width 0.6096) (layer F.Cu) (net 7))
 (segment (start 150.205 50.955) (end 150.205 48) (width 0.6096) (layer F.Cu) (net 7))
 (segment (start 150.25 51) (end 150.205 50.955) (width 0.6096) (layer F.Cu) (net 7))
 (via (at 150.25 51) (size 0.6858) (drill 0.3302) (layers F.Cu B.Cu) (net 7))
 (segment (start 171.5 51) (end 150.25 51) (width 0.6096) (layer B.Cu) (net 7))
 (segment (start 171.75 51.25) (end 171.5 51) (width 0.6096) (layer B.Cu) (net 7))
 (via (at 171.75 51.25) (size 0.6858) (drill 0.3302) (layers F.Cu B.Cu) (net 7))
 (segment (start 171.795 51.205) (end 171.75 51.25) (width 0.6096) (layer F.Cu) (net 7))
 (segment (start 145 40) (end 145 42.5) (width 0.3048) (layer B.Cu) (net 7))
 (segment (start 140.12 42.9) (end 142.1 42.9) (width 0.3048) (layer B.Cu) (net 7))
 (segment (start 142.1 42.9) (end 145 40) (width 0.3048) (layer B.Cu) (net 7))
 (segment (start 140.25 40.75) (end 140.25 42.77) (width 0.3048) (layer F.Cu) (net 7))
 (segment (start 140.25 42.77) (end 140.12 42.9) (width 0.3048) (layer F.Cu) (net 7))
 (segment (start 115.215076 42.315076) (end 116.3 43.4) (width 0.3048) (layer F.Cu) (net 2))
 (segment (start 114.9 52.3) (end 113.05 52.3) (width 0.3048) (layer F.Cu) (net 2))
 (segment (start 116.7 50.5) (end 114.9 52.3) (width 0.3048) (layer F.Cu) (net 2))
 (via (at 116.7 50.5) (size 0.6858) (drill 0.3302) (layers F.Cu B.Cu) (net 2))
 (segment (start 116.7 43.8) (end 116.7 50.5) (width 0.3048) (layer B.Cu) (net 2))
 (segment (start 116.3 43.4) (end 116.7 43.8) (width 0.3048) (layer B.Cu) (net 2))
 (via (at 116.3 43.4) (size 0.6858) (drill 0.3302) (layers F.Cu B.Cu) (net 2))
 (segment (start 115.215076 42.115076) (end 115.215076 42.315076) (width 0.3048) (layer F.Cu) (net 2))
 (segment (start 129 48) (end 132.48 48) (width 0.3048) (layer F.Cu) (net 8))
 (segment (start 132.48 48) (end 132.5 47.98) (width 0.3048) (layer F.Cu) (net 8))
 (segment (start 116.275736 41.054416) (end 116.275736 39.774264) (width 0.3048) (layer F.Cu) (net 1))
 (segment (start 116.275736 39.774264) (end 116.5 39.55) (width 0.3048) (layer F.Cu) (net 1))
 (segment (start 116.275736 39.674264) (end 116.5 39.45) (width 0.3048) (layer F.Cu) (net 1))
 (segment (start 116.781802 39.731802) (end 116.5 39.45) (width 0.3048) (layer F.Cu) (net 1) (status 30))
 (segment (start 114.154416 43.175736) (end 112.974264 43.175736) (width 0.3048) (layer F.Cu) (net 3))
 (segment (start 112.974264 43.175736) (end 112.55 43.6) (width 0.3048) (layer F.Cu) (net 3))
 (segment (start 112.8 43.5) (end 112.45 43.5) (width 0.3048) (layer F.Cu) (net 3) (status 30))
 (segment (start 118.114214 45.014214) (end 118.114214 45.114214) (width 0.3048) (layer F.Cu) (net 5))
 (segment (start 118.114214 45.114214) (end 121 48) (width 0.3048) (layer F.Cu) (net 5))
 (segment (start 145 48) (end 145 47) (width 0.3048) (layer B.Cu) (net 5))
 (segment (start 145 47) (end 142.25 44.25) (width 0.3048) (layer B.Cu) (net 5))
 (segment (start 124.25 44) (end 121 47.25) (width 0.3048) (layer B.Cu) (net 5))
 (via (at 124.25 44) (size 0.6858) (drill 0.3302) (layers F.Cu B.Cu) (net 5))
 (segment (start 125.75 44) (end 124.25 44) (width 0.3048) (layer F.Cu) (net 5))
 (via (at 125.75 44) (size 0.6858) (drill 0.3302) (layers F.Cu B.Cu) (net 5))
 (segment (start 126.75 44) (end 125.75 44) (width 0.3048) (layer B.Cu) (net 5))
 (segment (start 127 44.25) (end 126.75 44) (width 0.3048) (layer B.Cu) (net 5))
 (segment (start 142.25 44.25) (end 127 44.25) (width 0.3048) (layer B.Cu) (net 5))
 (segment (start 121 47.25) (end 121 48) (width 0.3048) (layer B.Cu) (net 5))
 (segment (start 140.12 47.98) (end 144.98 47.98) (width 0.3048) (layer B.Cu) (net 5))
 (segment (start 144.98 47.98) (end 145 48) (width 0.3048) (layer B.Cu) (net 5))
 (segment (start 144.98 47.98) (end 145 48) (width 0.3048) (layer F.Cu) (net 5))
 (segment (start 145 48) (end 145 47.4) (width 0.3048) (layer B.Cu) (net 5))
 (segment (start 121 46.1) (end 121 48) (width 0.3048) (layer B.Cu) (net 5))
 (segment (start 119.174874 43.953553) (end 119.174874 41.825126) (width 0.3048) (layer F.Cu) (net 6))
 (segment (start 119.174874 41.825126) (end 121 40) (width 0.3048) (layer F.Cu) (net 6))
 (segment (start 129 40) (end 129 40.75) (width 0.3048) (layer B.Cu) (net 6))
 (segment (start 129 40.75) (end 126.75 43) (width 0.3048) (layer B.Cu) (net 6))
 (segment (start 124.25 43) (end 121.25 40) (width 0.3048) (layer B.Cu) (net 6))
 (via (at 124.25 43) (size 0.6858) (drill 0.3302) (layers F.Cu B.Cu) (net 6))
 (segment (start 125.75 43) (end 124.25 43) (width 0.3048) (layer F.Cu) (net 6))
 (via (at 125.75 43) (size 0.6858) (drill 0.3302) (layers F.Cu B.Cu) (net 6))
 (segment (start 126.75 43) (end 125.75 43) (width 0.3048) (layer B.Cu) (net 6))
 (segment (start 121.25 40) (end 121 40) (width 0.3048) (layer B.Cu) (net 6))
 (segment (start 140.12 50.52) (end 139.08 50.52) (width 0.3048) (layer F.Cu) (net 6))
 (segment (start 132.5 40) (end 129 40) (width 0.3048) (layer F.Cu) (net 6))
 (segment (start 133.9 41.4) (end 132.5 40) (width 0.3048) (layer F.Cu) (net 6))
 (segment (start 133.9 49.6) (end 133.9 41.4) (width 0.3048) (layer F.Cu) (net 6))
 (segment (start 135.5 51.2) (end 133.9 49.6) (width 0.3048) (layer F.Cu) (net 6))
 (segment (start 138.4 51.2) (end 135.5 51.2) (width 0.3048) (layer F.Cu) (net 6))
 (segment (start 139.08 50.52) (end 138.4 51.2) (width 0.3048) (layer F.Cu) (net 6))
 (segment (start 118.873833 42.126167) (end 121 40) (width 0.3048) (layer F.Cu) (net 6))
 (segment (start 121 56) (end 120 56) (width 0.3048) (layer F.Cu) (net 4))
 (segment (start 120 56) (end 117.4 53.4) (width 0.3048) (layer F.Cu) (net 4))
 (segment (start 117.4 53.4) (end 117.4 46.421321) (width 0.3048) (layer F.Cu) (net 4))
 (segment (start 117.4 46.421321) (end 117.053553 46.074874) (width 0.3048) (layer F.Cu) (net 4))
 (segment (start 140.725 52.025) (end 126.775 52.025) (width 0.3048) (layer F.Cu) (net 4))
 (segment (start 123.25 51.25) (end 121 53.5) (width 0.3048) (layer F.Cu) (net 4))
 (segment (start 124 51.25) (end 123.25 51.25) (width 0.3048) (layer F.Cu) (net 4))
 (segment (start 124.25 51) (end 124 51.25) (width 0.3048) (layer F.Cu) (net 4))
 (via (at 124.25 51) (size 0.6858) (drill 0.3302) (layers F.Cu B.Cu) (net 4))
 (segment (start 125.75 51) (end 124.25 51) (width 0.3048) (layer B.Cu) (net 4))
 (via (at 125.75 51) (size 0.6858) (drill 0.3302) (layers F.Cu B.Cu) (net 4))
 (segment (start 126.775 52.025) (end 125.75 51) (width 0.3048) (layer F.Cu) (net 4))
 (segment (start 121 53.5) (end 121 56) (width 0.3048) (layer F.Cu) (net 4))
 (segment (start 145 56) (end 144.9 56) (width 0.3048) (layer F.Cu) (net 4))
 (segment (start 144.9 56) (end 141.4 52.5) (width 0.3048) (layer F.Cu) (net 4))
 (segment (start 141.4 46.72) (end 140.12 45.44) (width 0.3048) (layer F.Cu) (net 4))
 (segment (start 141.4 52.5) (end 141.4 46.72) (width 0.3048) (layer F.Cu) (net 4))
 (segment (start 145 56) (end 144.7 56) (width 0.3048) (layer F.Cu) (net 4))
 (segment (start 144.7 56) (end 140.725 52.025) (width 0.3048) (layer F.Cu) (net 4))
 (segment (start 140.725 52.025) (end 140.7 52) (width 0.3048) (layer F.Cu) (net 4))
 (segment (start 140.12 45.44) (end 139.84 45.44) (width 0.3048) (layer F.Cu) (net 4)))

